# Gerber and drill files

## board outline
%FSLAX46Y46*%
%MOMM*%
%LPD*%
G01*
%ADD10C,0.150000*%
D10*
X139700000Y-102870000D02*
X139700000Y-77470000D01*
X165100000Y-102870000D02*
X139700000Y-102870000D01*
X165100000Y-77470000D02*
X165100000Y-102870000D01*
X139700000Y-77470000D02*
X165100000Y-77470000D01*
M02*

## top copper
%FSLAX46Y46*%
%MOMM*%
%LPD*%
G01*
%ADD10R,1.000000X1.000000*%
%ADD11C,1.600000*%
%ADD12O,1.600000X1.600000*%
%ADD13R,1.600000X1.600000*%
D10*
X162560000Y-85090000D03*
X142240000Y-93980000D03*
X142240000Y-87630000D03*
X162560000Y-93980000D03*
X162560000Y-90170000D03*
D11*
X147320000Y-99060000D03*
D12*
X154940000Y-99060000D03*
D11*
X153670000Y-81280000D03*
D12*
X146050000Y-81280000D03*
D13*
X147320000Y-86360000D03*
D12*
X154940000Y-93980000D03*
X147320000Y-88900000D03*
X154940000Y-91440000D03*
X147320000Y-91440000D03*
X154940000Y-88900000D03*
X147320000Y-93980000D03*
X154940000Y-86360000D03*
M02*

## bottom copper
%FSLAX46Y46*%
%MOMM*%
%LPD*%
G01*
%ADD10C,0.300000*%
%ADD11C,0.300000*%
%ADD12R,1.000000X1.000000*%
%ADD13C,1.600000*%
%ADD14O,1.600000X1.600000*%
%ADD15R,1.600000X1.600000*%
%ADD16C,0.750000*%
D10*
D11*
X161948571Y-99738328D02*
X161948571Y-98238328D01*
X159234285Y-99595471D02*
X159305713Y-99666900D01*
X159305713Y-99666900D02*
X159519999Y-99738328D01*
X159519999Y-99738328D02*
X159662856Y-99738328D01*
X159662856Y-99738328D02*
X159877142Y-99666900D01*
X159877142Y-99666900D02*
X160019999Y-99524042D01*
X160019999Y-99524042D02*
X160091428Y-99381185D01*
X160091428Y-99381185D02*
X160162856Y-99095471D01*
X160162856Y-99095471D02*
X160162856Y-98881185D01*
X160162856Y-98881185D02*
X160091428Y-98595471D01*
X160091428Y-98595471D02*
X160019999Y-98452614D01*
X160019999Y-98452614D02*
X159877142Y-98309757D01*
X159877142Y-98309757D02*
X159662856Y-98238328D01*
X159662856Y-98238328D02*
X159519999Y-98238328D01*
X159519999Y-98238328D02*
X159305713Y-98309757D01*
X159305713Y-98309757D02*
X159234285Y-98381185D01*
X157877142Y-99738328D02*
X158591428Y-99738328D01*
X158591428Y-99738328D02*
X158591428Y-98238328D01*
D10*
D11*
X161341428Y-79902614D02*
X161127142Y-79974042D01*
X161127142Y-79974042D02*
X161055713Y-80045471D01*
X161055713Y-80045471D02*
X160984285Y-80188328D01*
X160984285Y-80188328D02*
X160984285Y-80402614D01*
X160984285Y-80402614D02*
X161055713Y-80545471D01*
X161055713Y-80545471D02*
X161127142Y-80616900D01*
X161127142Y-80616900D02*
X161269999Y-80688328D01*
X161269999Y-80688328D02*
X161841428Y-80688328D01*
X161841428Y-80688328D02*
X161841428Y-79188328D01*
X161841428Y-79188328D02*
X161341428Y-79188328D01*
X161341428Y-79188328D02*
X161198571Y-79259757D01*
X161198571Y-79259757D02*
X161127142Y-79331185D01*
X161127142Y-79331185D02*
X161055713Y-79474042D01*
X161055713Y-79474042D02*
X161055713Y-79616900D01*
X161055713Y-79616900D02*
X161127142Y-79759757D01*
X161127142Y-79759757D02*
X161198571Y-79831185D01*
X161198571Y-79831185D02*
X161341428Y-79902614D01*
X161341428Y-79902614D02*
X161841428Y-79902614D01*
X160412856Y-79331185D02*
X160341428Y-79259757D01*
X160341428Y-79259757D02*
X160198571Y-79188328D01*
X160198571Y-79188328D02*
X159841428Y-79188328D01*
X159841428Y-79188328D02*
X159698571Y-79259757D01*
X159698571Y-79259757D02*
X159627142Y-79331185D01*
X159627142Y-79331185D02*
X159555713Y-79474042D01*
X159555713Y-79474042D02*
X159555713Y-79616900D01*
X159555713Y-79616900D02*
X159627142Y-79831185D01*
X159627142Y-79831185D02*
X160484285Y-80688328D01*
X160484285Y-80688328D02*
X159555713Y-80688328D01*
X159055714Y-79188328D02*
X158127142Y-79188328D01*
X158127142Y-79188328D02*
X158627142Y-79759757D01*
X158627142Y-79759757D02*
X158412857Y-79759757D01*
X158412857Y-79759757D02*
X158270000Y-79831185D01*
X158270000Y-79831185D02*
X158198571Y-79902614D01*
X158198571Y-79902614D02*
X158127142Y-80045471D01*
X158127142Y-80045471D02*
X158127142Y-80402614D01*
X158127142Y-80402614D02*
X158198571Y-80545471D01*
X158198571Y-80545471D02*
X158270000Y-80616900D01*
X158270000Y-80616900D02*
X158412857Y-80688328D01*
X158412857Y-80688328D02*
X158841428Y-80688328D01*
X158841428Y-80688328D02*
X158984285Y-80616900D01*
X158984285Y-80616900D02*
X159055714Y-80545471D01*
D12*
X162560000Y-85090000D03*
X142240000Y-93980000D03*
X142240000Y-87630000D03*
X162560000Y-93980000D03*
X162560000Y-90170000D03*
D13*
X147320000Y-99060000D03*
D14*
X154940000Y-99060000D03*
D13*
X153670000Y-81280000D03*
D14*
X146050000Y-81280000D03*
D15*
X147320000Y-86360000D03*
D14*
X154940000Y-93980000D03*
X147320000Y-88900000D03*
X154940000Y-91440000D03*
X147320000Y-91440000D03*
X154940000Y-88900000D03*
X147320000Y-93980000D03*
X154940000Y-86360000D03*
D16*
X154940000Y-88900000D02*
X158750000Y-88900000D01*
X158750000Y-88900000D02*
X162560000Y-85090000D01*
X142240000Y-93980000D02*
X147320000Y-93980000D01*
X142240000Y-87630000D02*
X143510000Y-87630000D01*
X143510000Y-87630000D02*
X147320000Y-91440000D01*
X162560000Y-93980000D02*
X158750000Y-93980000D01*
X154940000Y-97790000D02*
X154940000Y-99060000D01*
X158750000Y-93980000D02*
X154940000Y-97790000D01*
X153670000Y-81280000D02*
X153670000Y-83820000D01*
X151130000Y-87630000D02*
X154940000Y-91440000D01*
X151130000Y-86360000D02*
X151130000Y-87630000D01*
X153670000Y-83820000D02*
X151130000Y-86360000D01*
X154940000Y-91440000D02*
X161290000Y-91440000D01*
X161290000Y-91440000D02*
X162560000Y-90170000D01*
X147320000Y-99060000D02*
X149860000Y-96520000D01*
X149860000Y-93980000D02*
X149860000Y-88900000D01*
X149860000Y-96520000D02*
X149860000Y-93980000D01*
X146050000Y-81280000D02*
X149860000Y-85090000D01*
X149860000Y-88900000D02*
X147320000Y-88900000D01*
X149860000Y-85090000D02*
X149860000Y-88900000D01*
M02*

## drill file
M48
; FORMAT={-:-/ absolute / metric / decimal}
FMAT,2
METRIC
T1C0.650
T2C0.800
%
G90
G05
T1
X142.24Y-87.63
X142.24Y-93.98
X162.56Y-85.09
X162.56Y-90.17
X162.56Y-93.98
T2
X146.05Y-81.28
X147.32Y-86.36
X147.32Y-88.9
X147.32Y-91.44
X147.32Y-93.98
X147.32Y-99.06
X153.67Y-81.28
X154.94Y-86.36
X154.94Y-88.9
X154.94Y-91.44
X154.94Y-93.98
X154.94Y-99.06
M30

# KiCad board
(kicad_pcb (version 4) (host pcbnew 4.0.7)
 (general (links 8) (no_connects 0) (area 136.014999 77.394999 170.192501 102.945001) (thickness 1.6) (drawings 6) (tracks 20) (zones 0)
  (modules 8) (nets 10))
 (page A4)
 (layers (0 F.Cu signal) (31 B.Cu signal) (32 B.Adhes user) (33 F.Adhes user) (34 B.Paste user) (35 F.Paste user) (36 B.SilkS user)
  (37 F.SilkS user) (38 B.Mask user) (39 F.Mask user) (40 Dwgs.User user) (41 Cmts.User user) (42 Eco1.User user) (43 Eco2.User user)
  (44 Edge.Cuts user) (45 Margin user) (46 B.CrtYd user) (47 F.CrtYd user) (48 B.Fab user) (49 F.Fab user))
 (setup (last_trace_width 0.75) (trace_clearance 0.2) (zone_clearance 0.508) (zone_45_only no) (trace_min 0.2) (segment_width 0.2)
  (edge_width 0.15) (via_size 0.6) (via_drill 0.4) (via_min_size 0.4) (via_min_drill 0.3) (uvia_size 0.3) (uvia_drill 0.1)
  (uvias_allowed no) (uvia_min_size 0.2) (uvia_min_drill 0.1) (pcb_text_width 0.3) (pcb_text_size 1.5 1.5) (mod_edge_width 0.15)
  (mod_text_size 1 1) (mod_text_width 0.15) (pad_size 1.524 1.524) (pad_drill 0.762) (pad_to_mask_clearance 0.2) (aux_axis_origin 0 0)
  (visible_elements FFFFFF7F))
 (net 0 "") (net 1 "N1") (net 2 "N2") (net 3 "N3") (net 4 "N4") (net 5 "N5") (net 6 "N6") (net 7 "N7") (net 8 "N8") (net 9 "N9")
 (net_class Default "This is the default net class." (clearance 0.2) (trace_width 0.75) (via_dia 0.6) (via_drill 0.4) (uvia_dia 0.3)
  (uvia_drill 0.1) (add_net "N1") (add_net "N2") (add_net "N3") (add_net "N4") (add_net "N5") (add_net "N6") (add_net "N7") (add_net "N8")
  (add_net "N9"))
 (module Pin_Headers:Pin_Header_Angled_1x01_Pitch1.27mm (layer F.Cu) (at 162.56 85.09)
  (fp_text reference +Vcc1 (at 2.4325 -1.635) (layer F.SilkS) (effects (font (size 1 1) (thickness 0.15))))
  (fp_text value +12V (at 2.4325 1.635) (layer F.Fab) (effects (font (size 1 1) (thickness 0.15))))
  (pad 1 thru_hole rect (at 0 0) (size 1 1) (drill 0.65) (layers *.Cu *.Mask) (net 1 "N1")))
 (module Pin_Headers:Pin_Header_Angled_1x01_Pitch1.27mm (layer F.Cu) (at 142.24 93.98 180)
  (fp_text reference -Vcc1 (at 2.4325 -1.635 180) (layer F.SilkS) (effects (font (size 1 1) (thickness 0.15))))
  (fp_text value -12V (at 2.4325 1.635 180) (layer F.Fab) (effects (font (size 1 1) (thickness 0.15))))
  (pad 1 thru_hole rect (at 0 0 180) (size 1 1) (drill 0.65) (layers *.Cu *.Mask) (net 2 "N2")))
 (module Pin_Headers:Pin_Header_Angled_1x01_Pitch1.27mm (layer F.Cu) (at 142.24 87.63 180)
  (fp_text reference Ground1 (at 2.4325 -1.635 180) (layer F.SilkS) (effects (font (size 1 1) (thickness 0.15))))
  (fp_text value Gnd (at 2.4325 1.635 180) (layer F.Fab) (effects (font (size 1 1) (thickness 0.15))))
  (pad 1 thru_hole rect (at 0 0 180) (size 1 1) (drill 0.65) (layers *.Cu *.Mask) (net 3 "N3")))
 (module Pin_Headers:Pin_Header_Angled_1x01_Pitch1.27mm (layer F.Cu) (at 162.56 93.98)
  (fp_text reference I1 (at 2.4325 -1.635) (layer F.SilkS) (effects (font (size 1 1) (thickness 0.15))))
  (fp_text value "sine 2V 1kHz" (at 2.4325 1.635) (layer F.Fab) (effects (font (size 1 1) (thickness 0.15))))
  (pad 1 thru_hole rect (at 0 0) (size 1 1) (drill 0.65) (layers *.Cu *.Mask) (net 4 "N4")))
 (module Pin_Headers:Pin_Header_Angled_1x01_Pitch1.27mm (layer F.Cu) (at 162.56 90.17)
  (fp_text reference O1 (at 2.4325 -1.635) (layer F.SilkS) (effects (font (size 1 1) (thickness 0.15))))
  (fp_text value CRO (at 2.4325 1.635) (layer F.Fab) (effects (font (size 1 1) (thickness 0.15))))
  (pad 1 thru_hole rect (at 0 0) (size 1 1) (drill 0.65) (layers *.Cu *.Mask) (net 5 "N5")))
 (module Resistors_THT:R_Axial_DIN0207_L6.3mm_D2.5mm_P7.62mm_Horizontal (layer F.Cu) (at 147.32 99.06)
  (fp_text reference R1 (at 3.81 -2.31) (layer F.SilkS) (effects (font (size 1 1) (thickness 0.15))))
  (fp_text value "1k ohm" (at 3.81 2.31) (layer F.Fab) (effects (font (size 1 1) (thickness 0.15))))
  (pad 1 thru_hole circle (at 0 0) (size 1.6 1.6) (drill 0.8) (layers *.Cu *.Mask) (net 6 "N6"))
  (pad 2 thru_hole oval (at 7.62 0) (size 1.6 1.6) (drill 0.8) (layers *.Cu *.Mask) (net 4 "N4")))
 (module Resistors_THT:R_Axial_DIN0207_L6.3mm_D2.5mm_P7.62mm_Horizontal (layer F.Cu) (at 153.67 81.28 180)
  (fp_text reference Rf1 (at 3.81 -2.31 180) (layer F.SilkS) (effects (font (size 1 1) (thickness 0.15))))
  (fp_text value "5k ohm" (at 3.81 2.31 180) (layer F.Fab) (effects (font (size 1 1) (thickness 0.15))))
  (pad 1 thru_hole circle (at 0 0 180) (size 1.6 1.6) (drill 0.8) (layers *.Cu *.Mask) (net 5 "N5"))
  (pad 2 thru_hole oval (at 7.62 0 180) (size 1.6 1.6) (drill 0.8) (layers *.Cu *.Mask) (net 6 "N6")))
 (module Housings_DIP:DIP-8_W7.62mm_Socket (layer F.Cu) (at 147.32 86.36)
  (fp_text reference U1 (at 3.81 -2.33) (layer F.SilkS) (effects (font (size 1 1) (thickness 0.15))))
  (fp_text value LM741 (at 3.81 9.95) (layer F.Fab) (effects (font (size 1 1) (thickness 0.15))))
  (pad 1 thru_hole rect (at 0 0) (size 1.6 1.6) (drill 0.8) (layers *.Cu *.Mask) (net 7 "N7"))
  (pad 5 thru_hole oval (at 7.62 7.62) (size 1.6 1.6) (drill 0.8) (layers *.Cu *.Mask) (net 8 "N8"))
  (pad 2 thru_hole oval (at 0 2.54) (size 1.6 1.6) (drill 0.8) (layers *.Cu *.Mask) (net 6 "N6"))
  (pad 6 thru_hole oval (at 7.62 5.08) (size 1.6 1.6) (drill 0.8) (layers *.Cu *.Mask) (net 5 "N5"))
  (pad 3 thru_hole oval (at 0 5.08) (size 1.6 1.6) (drill 0.8) (layers *.Cu *.Mask) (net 3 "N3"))
  (pad 7 thru_hole oval (at 7.62 2.54) (size 1.6 1.6) (drill 0.8) (layers *.Cu *.Mask) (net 1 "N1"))
  (pad 4 thru_hole oval (at 0 7.62) (size 1.6 1.6) (drill 0.8) (layers *.Cu *.Mask) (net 2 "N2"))
  (pad 8 thru_hole oval (at 7.62 0) (size 1.6 1.6) (drill 0.8) (layers *.Cu *.Mask) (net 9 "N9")))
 (gr_line (start 139.7 102.87) (end 139.7 77.47) (angle 90) (layer Edge.Cuts) (width 0.15))
 (gr_line (start 165.1 102.87) (end 139.7 102.87) (angle 90) (layer Edge.Cuts) (width 0.15))
 (gr_line (start 165.1 77.47) (end 165.1 102.87) (angle 90) (layer Edge.Cuts) (width 0.15))
 (gr_line (start 139.7 77.47) (end 165.1 77.47) (angle 90) (layer Edge.Cuts) (width 0.15))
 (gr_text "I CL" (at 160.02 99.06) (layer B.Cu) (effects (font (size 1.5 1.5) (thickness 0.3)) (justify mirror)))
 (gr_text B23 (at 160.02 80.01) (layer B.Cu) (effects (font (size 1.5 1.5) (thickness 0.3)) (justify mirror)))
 (segment (start 154.94 88.9) (end 158.75 88.9) (width 0.75) (layer B.Cu) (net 1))
 (segment (start 158.75 88.9) (end 162.56 85.09) (width 0.75) (layer B.Cu) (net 1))
 (segment (start 142.24 93.98) (end 147.32 93.98) (width 0.75) (layer B.Cu) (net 2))
 (segment (start 142.24 87.63) (end 143.51 87.63) (width 0.75) (layer B.Cu) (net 3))
 (segment (start 143.51 87.63) (end 147.32 91.44) (width 0.75) (layer B.Cu) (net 3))
 (segment (start 162.56 93.98) (end 158.75 93.98) (width 0.75) (layer B.Cu) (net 4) (status 400000))
 (segment (start 154.94 97.79) (end 154.94 99.06) (width 0.75) (layer B.Cu) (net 4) (status 800000))
 (segment (start 158.75 93.98) (end 154.94 97.79) (width 0.75) (layer B.Cu) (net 4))
 (segment (start 153.67 81.28) (end 153.67 83.82) (width 0.75) (layer B.Cu) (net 5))
 (segment (start 151.13 87.63) (end 154.94 91.44) (width 0.75) (layer B.Cu) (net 5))
 (segment (start 151.13 86.36) (end 151.13 87.63) (width 0.75) (layer B.Cu) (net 5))
 (segment (start 153.67 83.82) (end 151.13 86.36) (width 0.75) (layer B.Cu) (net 5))
 (segment (start 154.94 91.44) (end 161.29 91.44) (width 0.75) (layer B.Cu) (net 5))
 (segment (start 161.29 91.44) (end 162.56 90.17) (width 0.75) (layer B.Cu) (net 5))
 (segment (start 147.32 99.06) (end 149.86 96.52) (width 0.75) (layer B.Cu) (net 6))
 (segment (start 149.86 93.98) (end 149.86 88.9) (width 0.75) (layer B.Cu) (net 6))
 (segment (start 149.86 96.52) (end 149.86 93.98) (width 0.75) (layer B.Cu) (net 6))
 (segment (start 146.05 81.28) (end 149.86 85.09) (width 0.75) (layer B.Cu) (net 6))
 (segment (start 149.86 88.9) (end 147.32 88.9) (width 0.75) (layer B.Cu) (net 6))
 (segment (start 149.86 85.09) (end 149.86 88.9) (width 0.75) (layer B.Cu) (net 6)))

